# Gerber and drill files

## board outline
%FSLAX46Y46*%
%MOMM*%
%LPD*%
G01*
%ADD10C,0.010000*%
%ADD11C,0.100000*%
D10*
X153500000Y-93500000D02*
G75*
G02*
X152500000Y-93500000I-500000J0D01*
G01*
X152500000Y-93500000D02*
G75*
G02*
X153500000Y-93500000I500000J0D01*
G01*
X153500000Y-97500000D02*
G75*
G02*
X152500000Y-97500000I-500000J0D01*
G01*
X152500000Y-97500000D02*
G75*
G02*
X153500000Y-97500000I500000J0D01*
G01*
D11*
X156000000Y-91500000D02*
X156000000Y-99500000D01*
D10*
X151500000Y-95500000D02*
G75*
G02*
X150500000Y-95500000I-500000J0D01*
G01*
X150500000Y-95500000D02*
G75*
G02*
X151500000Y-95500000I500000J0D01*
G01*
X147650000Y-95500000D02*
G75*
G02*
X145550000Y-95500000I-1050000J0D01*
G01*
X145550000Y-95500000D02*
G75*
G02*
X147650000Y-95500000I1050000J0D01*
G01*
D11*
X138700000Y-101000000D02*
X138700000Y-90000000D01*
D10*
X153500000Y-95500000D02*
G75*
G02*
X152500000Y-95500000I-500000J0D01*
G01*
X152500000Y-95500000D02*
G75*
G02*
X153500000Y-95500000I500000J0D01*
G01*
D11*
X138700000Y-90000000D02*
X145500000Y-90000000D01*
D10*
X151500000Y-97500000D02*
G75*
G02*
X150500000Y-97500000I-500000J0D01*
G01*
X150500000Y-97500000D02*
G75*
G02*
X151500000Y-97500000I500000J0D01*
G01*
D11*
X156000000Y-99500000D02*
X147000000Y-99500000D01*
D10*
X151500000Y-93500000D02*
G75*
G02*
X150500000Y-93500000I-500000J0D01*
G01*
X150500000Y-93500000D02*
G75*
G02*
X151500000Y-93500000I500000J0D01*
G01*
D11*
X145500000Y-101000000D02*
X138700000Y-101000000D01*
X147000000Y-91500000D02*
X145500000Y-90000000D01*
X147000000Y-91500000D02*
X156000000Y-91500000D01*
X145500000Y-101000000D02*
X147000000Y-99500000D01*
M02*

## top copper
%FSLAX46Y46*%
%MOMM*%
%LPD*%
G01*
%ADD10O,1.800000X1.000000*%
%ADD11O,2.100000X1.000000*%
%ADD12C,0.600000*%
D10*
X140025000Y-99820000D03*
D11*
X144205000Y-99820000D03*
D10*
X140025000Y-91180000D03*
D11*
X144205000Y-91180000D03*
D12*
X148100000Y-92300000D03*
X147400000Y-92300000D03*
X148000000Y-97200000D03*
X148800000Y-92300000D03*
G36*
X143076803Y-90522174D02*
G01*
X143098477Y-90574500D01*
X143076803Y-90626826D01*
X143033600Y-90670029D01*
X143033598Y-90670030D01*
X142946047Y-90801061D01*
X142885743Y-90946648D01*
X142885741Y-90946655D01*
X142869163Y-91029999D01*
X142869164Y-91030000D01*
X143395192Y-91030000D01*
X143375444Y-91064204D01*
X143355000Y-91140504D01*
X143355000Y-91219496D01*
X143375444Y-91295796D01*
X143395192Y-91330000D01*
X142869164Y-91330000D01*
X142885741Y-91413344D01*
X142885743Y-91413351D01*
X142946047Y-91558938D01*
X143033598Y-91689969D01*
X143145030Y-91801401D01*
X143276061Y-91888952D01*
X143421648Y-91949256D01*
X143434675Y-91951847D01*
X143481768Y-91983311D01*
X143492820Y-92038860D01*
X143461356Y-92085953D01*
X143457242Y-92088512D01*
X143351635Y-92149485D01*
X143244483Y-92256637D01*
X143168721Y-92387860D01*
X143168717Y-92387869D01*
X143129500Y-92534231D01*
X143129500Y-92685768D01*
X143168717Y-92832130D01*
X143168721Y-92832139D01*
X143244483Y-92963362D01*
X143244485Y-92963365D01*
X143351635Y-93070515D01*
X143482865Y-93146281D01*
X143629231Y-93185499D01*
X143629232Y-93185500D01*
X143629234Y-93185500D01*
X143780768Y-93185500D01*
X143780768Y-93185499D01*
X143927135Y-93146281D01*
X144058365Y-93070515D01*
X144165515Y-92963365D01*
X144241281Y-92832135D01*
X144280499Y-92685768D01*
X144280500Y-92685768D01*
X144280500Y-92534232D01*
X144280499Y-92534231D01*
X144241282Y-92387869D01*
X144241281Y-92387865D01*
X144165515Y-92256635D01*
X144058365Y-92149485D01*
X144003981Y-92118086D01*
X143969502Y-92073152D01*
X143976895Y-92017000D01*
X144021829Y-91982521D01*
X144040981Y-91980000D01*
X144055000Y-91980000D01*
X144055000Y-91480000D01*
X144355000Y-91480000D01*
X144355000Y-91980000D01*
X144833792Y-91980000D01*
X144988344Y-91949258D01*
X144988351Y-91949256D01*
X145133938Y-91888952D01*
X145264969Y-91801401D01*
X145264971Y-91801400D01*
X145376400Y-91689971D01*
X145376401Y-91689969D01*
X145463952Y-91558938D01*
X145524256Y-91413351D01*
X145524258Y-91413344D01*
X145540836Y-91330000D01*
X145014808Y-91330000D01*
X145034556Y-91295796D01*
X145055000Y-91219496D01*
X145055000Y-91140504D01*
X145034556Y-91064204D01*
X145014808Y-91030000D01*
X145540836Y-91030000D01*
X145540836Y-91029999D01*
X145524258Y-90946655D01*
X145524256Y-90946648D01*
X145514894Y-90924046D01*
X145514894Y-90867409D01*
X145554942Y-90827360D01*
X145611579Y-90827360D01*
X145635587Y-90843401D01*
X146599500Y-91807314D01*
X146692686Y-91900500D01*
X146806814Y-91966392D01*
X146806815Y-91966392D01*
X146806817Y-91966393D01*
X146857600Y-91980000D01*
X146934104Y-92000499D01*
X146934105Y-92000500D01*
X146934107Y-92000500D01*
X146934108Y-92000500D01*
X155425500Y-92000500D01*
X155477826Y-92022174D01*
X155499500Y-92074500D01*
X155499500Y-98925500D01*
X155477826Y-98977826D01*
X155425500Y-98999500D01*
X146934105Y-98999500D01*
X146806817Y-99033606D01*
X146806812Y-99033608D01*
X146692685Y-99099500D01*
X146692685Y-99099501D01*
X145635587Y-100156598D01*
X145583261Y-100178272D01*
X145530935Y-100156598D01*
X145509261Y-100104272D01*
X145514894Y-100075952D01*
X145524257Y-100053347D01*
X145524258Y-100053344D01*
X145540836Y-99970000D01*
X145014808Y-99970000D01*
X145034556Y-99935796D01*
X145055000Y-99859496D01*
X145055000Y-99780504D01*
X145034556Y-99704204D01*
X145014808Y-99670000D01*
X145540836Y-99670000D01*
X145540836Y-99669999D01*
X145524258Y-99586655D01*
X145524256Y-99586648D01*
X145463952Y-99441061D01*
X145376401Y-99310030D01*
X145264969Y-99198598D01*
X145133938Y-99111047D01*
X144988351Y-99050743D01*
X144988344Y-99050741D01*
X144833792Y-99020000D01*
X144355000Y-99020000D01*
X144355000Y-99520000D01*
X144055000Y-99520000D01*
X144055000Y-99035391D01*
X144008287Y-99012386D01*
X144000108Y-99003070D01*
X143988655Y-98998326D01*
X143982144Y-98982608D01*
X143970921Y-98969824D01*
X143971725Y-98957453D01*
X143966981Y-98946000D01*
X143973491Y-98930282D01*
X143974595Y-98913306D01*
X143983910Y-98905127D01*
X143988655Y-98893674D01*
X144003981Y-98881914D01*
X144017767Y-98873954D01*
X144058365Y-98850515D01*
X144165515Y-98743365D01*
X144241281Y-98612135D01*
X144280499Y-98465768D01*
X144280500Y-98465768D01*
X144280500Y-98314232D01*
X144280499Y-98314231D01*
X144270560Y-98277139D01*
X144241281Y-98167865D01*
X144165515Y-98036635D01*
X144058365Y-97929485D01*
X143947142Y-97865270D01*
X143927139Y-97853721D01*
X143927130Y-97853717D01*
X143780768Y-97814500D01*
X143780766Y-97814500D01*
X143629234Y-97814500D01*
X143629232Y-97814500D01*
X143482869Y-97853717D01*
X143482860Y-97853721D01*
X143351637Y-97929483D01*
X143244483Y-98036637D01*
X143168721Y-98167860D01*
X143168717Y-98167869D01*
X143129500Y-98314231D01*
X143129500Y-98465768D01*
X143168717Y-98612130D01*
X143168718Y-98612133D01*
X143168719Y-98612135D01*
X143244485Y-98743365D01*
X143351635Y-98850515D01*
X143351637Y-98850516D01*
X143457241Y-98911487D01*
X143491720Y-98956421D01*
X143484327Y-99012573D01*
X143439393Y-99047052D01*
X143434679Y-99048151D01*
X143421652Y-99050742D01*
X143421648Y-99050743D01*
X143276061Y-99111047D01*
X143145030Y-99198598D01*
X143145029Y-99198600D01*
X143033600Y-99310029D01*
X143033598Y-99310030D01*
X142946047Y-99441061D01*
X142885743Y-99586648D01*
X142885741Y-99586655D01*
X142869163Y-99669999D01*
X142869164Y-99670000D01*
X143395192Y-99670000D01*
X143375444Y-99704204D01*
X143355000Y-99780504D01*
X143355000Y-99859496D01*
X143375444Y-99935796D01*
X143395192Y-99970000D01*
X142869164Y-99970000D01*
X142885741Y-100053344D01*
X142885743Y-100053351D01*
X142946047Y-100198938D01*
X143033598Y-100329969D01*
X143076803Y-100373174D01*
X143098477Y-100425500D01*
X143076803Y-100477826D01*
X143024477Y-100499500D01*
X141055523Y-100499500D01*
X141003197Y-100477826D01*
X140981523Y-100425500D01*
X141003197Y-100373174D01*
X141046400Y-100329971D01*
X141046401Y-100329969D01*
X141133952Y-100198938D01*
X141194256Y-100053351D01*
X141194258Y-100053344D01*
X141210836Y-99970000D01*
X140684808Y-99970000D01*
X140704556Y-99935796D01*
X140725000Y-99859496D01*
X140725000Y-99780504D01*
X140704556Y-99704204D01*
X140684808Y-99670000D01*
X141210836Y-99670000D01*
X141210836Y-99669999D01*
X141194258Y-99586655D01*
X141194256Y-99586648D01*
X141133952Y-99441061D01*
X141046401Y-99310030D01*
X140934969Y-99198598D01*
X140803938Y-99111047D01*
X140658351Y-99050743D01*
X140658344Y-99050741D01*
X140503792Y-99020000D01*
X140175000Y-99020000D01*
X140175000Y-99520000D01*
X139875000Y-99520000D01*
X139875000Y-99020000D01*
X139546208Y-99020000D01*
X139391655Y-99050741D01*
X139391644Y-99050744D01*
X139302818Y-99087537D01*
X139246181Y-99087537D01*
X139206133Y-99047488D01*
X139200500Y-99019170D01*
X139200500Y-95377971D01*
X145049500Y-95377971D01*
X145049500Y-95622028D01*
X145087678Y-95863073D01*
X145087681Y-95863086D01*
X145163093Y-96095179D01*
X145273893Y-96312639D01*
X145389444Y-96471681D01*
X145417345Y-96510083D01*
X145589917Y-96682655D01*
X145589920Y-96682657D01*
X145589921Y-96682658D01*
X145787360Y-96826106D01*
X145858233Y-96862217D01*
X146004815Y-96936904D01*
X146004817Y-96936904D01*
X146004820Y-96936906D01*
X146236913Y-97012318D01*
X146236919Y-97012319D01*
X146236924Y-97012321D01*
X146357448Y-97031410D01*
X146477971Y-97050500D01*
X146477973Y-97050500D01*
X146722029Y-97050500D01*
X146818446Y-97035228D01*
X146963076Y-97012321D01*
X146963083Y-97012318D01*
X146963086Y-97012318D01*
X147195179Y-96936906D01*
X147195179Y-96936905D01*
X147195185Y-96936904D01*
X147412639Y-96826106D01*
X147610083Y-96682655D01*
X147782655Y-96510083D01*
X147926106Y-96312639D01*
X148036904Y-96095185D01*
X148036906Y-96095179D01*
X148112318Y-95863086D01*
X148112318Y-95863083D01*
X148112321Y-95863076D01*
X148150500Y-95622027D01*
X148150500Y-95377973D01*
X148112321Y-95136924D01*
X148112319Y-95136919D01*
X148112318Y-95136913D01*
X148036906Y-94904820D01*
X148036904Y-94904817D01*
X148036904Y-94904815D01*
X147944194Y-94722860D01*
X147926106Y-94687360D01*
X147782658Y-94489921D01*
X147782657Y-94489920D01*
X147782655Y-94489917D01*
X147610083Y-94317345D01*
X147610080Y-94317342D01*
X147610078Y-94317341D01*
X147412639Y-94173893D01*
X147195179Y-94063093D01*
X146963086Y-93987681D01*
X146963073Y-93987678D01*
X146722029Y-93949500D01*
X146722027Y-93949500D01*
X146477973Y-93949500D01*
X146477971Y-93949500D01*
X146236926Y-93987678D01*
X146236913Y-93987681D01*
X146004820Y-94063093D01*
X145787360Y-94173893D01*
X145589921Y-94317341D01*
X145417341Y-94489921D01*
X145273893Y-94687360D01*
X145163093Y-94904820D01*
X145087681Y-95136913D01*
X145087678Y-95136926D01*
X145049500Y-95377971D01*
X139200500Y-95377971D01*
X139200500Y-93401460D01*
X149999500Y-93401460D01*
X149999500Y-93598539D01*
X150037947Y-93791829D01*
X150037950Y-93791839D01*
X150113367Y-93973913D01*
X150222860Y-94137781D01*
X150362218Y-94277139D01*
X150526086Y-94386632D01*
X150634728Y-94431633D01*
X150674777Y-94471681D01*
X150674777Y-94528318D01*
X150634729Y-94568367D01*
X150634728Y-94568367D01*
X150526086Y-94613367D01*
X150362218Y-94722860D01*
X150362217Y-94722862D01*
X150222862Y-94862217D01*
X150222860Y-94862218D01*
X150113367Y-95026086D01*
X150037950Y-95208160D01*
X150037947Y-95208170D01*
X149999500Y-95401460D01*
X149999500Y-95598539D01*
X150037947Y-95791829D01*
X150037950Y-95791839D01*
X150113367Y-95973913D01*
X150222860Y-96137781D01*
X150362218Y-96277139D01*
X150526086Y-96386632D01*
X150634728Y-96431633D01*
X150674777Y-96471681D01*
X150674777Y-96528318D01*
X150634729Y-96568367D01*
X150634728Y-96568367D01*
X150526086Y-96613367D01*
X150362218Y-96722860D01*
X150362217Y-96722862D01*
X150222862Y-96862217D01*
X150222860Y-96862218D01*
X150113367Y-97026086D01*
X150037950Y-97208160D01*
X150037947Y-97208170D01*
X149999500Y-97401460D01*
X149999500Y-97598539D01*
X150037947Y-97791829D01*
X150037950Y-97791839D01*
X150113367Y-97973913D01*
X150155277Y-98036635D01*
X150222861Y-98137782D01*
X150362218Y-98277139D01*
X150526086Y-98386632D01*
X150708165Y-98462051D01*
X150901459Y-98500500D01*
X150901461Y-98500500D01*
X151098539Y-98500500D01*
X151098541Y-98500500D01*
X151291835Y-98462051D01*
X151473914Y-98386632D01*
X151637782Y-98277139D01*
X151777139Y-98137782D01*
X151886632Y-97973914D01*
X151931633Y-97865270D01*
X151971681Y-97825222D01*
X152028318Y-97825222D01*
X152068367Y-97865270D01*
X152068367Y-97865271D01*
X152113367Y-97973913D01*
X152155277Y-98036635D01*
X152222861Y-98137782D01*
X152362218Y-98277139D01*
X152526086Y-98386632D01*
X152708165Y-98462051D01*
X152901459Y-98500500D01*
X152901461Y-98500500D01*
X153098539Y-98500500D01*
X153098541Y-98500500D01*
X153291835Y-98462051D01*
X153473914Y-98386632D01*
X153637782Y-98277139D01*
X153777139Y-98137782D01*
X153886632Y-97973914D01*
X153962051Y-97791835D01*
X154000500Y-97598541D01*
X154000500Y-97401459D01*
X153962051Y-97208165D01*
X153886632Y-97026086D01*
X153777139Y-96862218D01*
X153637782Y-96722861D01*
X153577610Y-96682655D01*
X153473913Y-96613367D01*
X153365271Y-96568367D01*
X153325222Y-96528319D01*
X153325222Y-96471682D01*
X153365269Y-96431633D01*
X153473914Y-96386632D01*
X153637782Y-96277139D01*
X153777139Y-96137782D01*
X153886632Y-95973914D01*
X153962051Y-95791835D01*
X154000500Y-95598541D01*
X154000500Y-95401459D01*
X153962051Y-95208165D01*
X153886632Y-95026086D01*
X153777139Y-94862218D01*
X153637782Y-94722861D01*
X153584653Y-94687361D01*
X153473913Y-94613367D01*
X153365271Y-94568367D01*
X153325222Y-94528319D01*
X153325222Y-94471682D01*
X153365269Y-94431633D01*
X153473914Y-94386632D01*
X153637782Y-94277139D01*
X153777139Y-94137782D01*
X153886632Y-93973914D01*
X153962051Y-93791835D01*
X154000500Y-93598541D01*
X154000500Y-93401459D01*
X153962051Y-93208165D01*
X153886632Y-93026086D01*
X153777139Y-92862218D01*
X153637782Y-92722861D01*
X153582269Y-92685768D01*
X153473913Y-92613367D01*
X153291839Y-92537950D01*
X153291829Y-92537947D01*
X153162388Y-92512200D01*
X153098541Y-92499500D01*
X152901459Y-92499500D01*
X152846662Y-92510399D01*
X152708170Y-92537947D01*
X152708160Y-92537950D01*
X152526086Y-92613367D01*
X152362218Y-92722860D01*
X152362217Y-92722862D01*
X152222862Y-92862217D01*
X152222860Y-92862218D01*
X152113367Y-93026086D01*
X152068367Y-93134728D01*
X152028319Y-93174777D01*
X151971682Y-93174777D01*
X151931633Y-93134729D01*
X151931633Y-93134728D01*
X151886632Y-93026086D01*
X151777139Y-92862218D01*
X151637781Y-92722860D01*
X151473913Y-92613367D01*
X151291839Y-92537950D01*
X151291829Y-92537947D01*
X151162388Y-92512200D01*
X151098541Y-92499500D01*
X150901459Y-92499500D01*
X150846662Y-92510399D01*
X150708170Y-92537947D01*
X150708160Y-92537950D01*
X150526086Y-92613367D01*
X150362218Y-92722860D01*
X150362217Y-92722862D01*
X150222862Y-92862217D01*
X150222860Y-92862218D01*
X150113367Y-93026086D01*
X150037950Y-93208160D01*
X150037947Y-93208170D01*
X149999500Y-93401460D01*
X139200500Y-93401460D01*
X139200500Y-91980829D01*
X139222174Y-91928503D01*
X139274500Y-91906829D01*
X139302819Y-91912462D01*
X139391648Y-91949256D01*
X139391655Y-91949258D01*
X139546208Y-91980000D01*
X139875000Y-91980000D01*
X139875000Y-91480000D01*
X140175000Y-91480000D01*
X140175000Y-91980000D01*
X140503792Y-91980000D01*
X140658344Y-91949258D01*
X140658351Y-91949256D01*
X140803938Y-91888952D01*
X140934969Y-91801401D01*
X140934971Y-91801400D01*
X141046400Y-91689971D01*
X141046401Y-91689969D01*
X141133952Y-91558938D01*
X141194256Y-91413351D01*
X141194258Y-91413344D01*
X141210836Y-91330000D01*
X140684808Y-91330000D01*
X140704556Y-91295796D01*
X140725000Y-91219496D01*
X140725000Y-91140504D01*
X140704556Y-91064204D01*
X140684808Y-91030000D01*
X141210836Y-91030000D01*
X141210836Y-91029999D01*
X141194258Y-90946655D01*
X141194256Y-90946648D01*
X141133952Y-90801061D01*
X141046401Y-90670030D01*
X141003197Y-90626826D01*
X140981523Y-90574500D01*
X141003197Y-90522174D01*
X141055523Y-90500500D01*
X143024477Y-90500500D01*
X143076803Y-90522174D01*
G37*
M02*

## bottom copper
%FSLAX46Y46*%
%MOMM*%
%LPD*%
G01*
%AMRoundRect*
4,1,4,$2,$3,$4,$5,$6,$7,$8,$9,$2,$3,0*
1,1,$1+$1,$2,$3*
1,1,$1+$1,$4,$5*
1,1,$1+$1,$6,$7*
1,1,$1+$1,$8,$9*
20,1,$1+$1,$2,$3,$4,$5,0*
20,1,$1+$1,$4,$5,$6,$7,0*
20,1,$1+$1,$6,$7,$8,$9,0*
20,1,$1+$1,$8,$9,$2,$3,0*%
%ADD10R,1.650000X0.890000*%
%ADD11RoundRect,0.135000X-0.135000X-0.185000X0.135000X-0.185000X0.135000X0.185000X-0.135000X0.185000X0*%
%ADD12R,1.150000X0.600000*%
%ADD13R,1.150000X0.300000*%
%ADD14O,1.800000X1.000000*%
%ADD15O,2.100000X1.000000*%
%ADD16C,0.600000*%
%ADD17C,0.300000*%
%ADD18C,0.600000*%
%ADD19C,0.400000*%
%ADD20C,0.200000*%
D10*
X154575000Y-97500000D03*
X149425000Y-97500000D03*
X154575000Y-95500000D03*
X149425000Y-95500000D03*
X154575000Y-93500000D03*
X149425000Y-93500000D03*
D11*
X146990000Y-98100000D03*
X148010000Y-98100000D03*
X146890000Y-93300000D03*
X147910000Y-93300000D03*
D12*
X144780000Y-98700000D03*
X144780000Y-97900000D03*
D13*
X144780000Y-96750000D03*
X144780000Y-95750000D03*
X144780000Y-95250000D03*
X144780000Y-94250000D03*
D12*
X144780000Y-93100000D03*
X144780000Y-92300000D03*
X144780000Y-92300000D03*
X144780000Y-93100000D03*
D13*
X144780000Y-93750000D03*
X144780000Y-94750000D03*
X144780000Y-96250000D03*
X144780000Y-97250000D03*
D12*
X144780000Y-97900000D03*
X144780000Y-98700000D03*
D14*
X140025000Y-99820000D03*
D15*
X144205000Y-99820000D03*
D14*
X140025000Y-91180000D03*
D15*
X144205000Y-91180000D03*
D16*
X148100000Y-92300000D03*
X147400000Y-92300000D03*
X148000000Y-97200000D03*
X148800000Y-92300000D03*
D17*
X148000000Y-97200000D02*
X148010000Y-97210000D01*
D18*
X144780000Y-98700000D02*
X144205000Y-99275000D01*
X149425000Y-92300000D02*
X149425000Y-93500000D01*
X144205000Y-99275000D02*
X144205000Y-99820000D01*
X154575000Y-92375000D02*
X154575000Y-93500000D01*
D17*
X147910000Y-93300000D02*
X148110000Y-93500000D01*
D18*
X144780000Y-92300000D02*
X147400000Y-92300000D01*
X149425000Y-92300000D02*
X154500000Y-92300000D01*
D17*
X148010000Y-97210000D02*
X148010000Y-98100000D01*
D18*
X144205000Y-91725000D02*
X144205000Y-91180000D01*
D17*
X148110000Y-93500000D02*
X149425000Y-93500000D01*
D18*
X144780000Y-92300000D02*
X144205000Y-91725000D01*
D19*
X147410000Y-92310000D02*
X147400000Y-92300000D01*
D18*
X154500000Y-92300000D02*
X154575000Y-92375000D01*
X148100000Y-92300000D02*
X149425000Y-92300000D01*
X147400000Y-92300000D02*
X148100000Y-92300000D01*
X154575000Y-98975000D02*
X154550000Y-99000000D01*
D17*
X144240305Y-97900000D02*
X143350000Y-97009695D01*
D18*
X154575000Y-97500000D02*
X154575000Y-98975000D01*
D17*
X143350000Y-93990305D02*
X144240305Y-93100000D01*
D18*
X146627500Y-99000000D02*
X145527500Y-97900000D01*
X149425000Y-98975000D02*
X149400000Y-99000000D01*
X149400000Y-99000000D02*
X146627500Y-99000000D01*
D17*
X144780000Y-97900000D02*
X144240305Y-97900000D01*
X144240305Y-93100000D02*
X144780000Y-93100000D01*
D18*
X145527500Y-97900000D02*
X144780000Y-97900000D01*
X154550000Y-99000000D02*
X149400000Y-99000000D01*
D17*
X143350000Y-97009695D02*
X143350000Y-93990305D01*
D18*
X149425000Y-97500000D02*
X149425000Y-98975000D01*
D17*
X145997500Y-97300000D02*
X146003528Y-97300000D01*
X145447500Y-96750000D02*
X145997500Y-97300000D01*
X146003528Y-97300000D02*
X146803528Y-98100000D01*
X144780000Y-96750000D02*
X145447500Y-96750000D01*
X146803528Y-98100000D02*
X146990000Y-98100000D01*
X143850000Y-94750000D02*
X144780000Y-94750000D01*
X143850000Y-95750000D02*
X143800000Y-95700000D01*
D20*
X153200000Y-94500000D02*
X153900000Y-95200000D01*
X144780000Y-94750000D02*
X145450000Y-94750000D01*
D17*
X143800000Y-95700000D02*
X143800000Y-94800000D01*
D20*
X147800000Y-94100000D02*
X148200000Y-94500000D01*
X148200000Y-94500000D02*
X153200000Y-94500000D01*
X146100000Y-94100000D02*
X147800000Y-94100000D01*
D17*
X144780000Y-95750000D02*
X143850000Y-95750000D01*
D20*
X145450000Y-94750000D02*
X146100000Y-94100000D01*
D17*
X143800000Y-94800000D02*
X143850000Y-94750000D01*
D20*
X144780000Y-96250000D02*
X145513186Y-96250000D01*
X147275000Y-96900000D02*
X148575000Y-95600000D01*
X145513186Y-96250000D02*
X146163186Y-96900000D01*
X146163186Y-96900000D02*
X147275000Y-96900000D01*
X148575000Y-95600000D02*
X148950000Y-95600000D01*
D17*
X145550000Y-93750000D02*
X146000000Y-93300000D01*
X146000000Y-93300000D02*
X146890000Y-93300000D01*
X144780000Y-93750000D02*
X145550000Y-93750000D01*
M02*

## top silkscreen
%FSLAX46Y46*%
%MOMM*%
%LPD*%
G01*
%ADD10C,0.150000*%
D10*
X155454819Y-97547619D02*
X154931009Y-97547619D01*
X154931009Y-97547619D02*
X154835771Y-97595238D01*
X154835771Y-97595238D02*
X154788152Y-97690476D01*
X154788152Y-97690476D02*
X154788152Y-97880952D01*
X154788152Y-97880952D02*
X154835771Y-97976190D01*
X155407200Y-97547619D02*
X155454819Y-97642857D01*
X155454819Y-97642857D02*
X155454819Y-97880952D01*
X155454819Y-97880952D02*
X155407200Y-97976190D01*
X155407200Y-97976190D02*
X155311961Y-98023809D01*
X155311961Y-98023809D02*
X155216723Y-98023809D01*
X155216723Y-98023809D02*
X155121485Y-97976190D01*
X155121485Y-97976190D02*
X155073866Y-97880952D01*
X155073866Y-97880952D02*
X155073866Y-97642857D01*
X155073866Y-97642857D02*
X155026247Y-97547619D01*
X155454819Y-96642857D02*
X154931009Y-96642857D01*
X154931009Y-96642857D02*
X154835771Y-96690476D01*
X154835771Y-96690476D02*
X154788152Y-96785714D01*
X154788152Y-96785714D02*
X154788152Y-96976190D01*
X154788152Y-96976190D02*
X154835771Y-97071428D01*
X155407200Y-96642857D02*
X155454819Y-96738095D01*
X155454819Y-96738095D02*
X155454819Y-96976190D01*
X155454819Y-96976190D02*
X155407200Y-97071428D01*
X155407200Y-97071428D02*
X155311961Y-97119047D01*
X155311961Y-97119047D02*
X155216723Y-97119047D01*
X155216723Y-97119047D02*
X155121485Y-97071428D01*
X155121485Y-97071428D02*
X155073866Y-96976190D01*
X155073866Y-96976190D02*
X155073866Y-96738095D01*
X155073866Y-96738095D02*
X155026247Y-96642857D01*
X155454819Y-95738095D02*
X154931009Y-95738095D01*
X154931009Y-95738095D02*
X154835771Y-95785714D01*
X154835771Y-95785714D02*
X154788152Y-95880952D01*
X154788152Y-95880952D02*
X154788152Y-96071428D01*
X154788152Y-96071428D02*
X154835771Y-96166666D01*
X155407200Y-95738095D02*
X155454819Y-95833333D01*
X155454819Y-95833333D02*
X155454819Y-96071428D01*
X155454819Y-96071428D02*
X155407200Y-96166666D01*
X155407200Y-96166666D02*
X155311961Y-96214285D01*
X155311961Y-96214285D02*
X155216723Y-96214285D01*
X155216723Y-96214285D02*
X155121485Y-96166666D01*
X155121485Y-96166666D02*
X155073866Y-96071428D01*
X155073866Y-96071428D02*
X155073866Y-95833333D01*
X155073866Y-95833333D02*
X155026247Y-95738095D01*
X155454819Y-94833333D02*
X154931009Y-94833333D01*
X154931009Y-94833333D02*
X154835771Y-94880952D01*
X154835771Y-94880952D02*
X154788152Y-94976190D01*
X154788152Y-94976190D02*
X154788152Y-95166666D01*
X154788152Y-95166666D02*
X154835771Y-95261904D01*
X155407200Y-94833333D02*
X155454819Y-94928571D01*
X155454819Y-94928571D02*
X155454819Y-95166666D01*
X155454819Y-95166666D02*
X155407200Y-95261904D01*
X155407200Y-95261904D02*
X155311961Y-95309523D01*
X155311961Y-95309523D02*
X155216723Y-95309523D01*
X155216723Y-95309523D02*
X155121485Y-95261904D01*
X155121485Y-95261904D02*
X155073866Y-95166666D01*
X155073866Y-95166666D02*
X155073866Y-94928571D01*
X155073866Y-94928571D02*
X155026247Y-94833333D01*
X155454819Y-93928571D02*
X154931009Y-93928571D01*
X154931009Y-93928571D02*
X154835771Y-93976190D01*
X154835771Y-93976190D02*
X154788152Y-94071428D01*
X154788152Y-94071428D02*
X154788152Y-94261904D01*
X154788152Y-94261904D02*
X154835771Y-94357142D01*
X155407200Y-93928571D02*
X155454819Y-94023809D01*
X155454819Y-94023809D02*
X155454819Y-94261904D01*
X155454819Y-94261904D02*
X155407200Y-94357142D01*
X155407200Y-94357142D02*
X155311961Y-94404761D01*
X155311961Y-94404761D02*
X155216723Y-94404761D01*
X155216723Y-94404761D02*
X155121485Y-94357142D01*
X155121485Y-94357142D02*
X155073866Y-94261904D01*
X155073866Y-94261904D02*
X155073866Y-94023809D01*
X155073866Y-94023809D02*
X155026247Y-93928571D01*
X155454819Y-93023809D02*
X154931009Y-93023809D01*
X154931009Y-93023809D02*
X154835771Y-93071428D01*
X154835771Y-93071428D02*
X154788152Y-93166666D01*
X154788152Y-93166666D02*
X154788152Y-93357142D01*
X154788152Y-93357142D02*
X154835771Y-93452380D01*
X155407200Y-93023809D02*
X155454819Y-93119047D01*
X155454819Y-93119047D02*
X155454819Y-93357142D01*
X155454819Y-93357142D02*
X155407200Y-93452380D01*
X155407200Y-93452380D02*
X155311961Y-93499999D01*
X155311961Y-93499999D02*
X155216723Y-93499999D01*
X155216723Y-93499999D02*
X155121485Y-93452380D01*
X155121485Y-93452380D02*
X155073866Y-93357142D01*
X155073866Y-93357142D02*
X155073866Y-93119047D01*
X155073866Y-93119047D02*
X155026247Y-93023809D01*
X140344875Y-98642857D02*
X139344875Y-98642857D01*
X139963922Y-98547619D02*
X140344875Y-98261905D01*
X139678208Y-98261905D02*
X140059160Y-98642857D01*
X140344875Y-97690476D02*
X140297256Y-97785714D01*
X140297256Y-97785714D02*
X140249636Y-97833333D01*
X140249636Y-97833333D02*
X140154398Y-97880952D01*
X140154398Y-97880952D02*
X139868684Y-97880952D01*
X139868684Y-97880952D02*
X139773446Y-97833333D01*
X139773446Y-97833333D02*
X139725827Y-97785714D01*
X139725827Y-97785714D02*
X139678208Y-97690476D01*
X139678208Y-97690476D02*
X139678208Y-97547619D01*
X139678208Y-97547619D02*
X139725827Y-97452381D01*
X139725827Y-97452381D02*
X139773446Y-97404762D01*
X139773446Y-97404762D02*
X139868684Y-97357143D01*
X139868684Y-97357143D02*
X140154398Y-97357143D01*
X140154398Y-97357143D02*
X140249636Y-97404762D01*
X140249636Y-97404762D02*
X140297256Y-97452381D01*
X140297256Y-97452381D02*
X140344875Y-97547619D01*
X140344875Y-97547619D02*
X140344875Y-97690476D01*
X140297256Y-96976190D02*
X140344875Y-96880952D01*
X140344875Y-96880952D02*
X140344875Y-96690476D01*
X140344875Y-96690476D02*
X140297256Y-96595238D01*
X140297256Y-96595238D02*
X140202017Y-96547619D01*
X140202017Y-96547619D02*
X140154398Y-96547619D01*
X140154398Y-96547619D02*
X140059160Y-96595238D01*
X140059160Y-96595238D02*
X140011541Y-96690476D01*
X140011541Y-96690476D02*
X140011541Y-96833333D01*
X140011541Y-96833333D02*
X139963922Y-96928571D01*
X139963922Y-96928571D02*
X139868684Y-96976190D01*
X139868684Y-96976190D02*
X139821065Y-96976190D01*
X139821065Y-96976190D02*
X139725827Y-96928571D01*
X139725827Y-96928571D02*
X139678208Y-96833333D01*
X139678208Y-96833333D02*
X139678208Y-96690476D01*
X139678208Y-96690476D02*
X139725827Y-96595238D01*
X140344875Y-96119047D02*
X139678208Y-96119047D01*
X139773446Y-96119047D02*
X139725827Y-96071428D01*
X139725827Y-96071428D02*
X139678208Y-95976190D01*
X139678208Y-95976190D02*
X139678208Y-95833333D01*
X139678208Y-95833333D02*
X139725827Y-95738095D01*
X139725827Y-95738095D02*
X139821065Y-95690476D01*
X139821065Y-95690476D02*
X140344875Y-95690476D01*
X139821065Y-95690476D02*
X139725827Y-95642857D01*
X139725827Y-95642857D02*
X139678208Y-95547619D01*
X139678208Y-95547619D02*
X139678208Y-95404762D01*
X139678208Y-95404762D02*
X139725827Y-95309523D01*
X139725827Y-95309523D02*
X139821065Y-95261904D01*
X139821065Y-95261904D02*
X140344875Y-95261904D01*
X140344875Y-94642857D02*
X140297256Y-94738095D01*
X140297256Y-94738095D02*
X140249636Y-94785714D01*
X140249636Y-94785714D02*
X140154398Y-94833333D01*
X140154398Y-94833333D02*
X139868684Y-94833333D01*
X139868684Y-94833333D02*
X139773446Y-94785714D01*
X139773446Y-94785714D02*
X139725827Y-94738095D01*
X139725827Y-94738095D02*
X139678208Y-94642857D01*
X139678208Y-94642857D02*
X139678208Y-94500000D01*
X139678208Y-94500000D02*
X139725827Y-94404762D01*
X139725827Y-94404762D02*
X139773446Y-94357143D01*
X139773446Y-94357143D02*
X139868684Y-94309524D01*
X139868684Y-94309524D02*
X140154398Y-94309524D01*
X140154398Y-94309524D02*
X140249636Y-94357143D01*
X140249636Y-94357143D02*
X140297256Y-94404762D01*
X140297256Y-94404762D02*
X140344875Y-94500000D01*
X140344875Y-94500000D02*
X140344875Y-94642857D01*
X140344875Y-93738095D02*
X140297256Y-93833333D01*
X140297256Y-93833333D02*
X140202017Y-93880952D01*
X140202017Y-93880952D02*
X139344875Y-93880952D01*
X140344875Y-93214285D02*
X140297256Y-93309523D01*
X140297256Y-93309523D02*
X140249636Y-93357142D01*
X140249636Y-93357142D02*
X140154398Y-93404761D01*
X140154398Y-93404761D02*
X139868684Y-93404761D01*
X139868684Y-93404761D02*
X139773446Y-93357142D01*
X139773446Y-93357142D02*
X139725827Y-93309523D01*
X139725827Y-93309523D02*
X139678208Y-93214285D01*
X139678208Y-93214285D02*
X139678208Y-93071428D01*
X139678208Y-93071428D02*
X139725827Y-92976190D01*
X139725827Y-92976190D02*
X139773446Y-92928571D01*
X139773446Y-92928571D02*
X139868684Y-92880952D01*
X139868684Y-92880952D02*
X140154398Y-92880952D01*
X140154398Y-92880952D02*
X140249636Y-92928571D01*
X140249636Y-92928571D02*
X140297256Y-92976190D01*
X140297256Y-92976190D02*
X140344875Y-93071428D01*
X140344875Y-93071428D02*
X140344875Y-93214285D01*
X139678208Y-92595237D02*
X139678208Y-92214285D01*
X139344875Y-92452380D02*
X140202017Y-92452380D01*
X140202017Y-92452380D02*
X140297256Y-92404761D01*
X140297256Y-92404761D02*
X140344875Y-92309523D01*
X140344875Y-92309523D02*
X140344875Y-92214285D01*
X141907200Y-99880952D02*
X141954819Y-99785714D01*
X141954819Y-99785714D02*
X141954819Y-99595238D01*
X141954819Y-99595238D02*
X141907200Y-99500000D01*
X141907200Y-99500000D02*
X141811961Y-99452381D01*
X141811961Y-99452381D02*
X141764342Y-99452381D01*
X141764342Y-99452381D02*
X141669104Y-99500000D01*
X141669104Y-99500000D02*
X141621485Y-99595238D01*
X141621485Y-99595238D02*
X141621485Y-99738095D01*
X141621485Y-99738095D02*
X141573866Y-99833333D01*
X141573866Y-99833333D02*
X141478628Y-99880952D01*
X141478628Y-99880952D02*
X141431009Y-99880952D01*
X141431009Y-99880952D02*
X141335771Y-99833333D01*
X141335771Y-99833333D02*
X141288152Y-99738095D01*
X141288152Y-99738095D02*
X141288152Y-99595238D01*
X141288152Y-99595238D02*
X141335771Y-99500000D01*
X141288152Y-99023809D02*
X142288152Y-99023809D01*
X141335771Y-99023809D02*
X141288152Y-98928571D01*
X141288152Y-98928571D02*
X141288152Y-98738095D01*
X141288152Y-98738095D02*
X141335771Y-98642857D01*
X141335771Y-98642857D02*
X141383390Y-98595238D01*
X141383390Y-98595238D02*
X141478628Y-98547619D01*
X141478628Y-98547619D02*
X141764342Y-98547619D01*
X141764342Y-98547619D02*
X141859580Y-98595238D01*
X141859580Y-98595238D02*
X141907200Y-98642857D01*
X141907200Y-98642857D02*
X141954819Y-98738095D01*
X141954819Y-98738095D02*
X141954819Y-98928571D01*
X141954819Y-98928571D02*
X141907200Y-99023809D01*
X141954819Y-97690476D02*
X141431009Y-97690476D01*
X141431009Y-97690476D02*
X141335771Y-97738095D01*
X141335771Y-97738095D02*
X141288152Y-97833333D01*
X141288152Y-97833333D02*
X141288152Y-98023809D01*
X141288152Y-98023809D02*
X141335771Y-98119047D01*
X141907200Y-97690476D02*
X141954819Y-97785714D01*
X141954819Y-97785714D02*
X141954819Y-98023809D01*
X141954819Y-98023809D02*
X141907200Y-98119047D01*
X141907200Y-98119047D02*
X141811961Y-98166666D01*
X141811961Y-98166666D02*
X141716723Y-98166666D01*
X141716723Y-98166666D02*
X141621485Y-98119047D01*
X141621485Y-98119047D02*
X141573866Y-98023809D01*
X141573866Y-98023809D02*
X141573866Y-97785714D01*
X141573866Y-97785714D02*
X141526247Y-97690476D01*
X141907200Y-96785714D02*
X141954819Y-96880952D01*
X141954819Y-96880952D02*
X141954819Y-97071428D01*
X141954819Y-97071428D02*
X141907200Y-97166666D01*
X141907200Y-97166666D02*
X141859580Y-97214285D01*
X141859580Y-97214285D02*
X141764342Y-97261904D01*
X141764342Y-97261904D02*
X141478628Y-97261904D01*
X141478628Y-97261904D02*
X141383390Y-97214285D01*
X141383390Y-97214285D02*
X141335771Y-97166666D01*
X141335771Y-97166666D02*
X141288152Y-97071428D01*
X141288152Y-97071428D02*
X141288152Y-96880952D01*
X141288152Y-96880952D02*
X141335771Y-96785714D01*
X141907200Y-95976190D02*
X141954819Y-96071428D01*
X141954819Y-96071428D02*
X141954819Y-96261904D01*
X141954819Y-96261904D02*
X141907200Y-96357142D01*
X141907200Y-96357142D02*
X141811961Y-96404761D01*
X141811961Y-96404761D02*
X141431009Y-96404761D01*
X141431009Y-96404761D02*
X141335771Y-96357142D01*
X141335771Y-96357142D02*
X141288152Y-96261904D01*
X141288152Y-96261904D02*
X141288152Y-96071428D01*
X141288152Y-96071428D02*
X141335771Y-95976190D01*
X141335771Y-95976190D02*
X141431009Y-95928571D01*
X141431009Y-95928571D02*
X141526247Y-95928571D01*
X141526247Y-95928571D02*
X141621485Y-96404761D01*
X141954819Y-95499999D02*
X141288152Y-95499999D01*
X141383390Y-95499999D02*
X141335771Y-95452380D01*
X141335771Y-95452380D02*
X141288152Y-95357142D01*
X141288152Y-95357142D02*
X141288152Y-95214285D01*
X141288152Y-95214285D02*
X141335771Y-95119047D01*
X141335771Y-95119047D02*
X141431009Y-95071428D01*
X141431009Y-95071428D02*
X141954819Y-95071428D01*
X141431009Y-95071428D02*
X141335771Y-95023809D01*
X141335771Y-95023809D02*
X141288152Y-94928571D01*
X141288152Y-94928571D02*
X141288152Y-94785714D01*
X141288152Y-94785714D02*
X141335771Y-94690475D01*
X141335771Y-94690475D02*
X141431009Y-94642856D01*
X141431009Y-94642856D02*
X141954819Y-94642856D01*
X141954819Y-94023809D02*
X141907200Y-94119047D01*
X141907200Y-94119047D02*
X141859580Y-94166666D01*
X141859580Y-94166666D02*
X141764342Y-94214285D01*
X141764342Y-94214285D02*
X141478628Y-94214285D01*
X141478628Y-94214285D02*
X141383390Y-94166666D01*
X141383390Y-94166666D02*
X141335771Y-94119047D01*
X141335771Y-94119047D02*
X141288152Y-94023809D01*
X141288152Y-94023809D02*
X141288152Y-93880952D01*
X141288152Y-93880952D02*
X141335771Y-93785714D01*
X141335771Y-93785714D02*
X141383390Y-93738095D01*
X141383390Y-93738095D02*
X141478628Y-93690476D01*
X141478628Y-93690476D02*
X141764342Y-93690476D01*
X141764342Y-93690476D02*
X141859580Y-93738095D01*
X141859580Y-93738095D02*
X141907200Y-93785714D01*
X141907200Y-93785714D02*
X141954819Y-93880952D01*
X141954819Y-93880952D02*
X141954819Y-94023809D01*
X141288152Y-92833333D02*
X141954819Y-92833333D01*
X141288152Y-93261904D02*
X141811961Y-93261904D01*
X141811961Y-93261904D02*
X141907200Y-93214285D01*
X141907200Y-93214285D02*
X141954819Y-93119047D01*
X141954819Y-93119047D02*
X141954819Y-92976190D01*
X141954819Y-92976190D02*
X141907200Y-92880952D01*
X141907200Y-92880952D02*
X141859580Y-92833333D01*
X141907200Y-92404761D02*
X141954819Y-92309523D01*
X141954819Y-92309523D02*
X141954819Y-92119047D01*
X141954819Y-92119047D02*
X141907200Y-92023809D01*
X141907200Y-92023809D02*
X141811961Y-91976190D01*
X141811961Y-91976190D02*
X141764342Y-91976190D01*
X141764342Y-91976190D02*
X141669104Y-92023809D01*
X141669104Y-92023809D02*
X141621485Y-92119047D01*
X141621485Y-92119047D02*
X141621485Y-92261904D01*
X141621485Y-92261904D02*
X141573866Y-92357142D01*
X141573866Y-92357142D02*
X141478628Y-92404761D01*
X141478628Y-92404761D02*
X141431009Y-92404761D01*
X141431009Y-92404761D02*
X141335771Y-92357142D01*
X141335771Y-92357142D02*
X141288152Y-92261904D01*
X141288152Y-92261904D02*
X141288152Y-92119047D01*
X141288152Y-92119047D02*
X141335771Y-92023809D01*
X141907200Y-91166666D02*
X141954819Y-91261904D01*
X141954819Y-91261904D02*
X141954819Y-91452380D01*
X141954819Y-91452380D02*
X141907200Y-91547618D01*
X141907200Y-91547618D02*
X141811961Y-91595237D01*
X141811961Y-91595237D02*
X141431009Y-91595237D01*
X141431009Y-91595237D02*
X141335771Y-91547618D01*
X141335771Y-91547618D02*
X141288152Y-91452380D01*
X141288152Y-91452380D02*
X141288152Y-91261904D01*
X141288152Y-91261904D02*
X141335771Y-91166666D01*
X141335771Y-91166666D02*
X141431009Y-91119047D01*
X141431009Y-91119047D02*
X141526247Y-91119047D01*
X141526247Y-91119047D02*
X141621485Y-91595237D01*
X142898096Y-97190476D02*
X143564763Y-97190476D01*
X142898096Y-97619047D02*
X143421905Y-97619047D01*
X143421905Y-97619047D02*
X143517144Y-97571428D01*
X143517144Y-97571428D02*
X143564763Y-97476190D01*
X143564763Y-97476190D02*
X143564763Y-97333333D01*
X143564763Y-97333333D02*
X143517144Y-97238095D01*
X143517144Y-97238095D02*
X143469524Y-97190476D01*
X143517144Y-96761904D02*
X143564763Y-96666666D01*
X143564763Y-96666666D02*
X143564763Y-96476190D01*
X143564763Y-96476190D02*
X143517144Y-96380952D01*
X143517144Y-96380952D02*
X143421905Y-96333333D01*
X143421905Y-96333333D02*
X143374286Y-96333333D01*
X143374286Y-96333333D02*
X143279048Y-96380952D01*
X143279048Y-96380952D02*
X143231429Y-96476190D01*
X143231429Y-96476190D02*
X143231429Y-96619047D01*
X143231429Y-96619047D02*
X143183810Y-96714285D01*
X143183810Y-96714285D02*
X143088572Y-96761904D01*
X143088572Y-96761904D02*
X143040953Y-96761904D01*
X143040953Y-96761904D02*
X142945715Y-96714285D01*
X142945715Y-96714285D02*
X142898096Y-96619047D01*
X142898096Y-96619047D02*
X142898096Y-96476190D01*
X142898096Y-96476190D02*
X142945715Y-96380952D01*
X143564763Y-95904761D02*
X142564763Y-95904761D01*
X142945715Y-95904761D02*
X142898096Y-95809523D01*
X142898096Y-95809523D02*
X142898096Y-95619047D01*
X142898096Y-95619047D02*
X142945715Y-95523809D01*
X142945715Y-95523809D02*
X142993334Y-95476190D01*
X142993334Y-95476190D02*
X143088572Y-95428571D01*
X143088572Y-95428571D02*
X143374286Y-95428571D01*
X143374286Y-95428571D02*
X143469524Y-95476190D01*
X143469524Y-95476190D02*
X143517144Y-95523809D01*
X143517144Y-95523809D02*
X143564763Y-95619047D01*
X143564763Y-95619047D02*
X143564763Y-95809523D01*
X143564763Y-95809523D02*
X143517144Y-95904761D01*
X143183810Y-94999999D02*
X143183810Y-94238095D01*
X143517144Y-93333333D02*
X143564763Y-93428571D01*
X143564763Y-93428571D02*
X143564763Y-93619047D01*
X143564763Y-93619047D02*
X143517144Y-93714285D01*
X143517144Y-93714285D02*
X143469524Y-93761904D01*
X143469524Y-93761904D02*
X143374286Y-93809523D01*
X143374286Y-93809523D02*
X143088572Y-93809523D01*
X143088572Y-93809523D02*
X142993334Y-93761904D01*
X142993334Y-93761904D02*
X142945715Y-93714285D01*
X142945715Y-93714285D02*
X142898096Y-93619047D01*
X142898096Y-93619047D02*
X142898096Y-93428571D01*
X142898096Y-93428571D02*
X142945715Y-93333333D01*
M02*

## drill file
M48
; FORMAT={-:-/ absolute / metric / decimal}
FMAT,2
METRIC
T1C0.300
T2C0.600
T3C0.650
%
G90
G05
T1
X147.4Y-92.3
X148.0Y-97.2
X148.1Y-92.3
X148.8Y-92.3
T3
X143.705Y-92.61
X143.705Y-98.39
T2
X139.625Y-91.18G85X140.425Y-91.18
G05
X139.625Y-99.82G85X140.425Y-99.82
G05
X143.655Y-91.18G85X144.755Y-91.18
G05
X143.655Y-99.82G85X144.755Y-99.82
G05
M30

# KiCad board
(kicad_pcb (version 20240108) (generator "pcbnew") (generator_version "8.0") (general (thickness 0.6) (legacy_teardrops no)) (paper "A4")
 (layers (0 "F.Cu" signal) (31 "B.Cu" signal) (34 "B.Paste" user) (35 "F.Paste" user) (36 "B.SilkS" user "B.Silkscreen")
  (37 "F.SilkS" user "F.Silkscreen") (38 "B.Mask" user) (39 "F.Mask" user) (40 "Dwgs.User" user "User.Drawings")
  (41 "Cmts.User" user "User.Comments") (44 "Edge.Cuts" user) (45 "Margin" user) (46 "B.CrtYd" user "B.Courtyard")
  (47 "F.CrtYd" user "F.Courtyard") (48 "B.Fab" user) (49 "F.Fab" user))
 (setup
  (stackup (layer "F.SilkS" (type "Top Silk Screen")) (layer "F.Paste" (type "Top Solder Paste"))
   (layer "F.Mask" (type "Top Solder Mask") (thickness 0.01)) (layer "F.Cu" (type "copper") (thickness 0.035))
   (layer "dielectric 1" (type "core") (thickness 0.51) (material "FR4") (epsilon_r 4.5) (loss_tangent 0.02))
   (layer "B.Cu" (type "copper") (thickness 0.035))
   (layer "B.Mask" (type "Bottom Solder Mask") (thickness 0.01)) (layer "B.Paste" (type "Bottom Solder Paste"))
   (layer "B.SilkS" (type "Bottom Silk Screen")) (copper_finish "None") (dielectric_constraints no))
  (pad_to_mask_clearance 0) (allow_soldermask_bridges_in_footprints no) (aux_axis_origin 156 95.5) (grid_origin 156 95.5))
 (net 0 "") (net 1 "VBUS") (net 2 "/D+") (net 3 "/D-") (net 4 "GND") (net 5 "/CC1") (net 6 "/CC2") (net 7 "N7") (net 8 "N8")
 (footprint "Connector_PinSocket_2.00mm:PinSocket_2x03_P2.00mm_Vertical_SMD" (layer "B.Cu") (at 152 95.5)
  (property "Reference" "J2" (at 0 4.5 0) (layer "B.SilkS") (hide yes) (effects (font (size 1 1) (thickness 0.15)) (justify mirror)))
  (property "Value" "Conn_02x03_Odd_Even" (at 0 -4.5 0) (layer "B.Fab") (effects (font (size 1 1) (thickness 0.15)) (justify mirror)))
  (pad "1" smd rect (at 2.575 2) (size 1.65 0.89) (layers "B.Cu" "B.Paste" "B.Mask") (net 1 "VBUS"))
  (pad "2" smd rect (at -2.575 2) (size 1.65 0.89) (layers "B.Cu" "B.Paste" "B.Mask") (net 1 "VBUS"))
  (pad "3" smd rect (at 2.575 0) (size 1.65 0.89) (layers "B.Cu" "B.Paste" "B.Mask") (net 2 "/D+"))
  (pad "4" smd rect (at -2.575 0) (size 1.65 0.89) (layers "B.Cu" "B.Paste" "B.Mask") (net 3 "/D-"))
  (pad "5" smd rect (at 2.575 -2) (size 1.65 0.89) (layers "B.Cu" "B.Paste" "B.Mask") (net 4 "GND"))
  (pad "6" smd rect (at -2.575 -2) (size 1.65 0.89) (layers "B.Cu" "B.Paste" "B.Mask") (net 4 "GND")))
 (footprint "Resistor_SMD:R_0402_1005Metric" (layer "B.Cu") (at 147.5 98.1)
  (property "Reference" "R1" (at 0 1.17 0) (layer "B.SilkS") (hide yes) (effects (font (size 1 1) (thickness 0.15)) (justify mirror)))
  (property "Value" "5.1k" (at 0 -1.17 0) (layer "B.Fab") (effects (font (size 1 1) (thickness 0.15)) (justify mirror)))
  (pad "1" smd roundrect (at -0.51 0) (size 0.54 0.64) (layers "B.Cu" "B.Paste" "B.Mask") (roundrect_rratio 0.25) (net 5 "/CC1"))
  (pad "2" smd roundrect (at 0.51 0) (size 0.54 0.64) (layers "B.Cu" "B.Paste" "B.Mask") (roundrect_rratio 0.25) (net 4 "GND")))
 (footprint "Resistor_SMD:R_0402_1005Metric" (layer "B.Cu") (at 147.4 93.3)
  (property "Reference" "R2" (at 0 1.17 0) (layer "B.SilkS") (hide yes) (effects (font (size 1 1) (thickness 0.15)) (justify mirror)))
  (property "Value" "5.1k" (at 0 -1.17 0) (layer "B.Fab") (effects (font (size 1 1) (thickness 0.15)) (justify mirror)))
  (pad "1" smd roundrect (at -0.51 0) (size 0.54 0.64) (layers "B.Cu" "B.Paste" "B.Mask") (roundrect_rratio 0.25) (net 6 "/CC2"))
  (pad "2" smd roundrect (at 0.51 0) (size 0.54 0.64) (layers "B.Cu" "B.Paste" "B.Mask") (roundrect_rratio 0.25) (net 4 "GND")))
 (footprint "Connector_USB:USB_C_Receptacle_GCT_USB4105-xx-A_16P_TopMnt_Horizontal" (layer "B.Cu") (at 141.1 95.5 90)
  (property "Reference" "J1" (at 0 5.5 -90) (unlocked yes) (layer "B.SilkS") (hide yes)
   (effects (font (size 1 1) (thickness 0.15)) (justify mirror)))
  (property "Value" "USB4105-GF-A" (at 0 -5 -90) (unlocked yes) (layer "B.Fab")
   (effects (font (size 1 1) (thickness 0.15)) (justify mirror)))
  (pad "" np_thru_hole circle (at -2.89 2.605 90) (size 0.65 0.65) (drill 0.65) (layers "F&B.Cu" "*.Mask"))
  (pad "" np_thru_hole circle (at 2.89 2.605 90) (size 0.65 0.65) (drill 0.65) (layers "F&B.Cu" "*.Mask"))
  (pad "A1" smd rect (at -3.2 3.68 90) (size 0.6 1.15) (layers "B.Cu" "B.Paste" "B.Mask") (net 4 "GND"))
  (pad "A4" smd rect (at -2.4 3.68 90) (size 0.6 1.15) (layers "B.Cu" "B.Paste" "B.Mask") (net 1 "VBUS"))
  (pad "A5" smd rect (at -1.25 3.68 90) (size 0.3 1.15) (layers "B.Cu" "B.Paste" "B.Mask") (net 5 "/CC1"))
  (pad "A6" smd rect (at -0.25 3.68 90) (size 0.3 1.15) (layers "B.Cu" "B.Paste" "B.Mask") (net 2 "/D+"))
  (pad "A7" smd rect (at 0.25 3.68 90) (size 0.3 1.15) (layers "B.Cu" "B.Paste" "B.Mask") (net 3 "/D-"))
  (pad "A8" smd rect (at 1.25 3.68 90) (size 0.3 1.15) (layers "B.Cu" "B.Paste" "B.Mask") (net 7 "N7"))
  (pad "A9" smd rect (at 2.4 3.68 90) (size 0.6 1.15) (layers "B.Cu" "B.Paste" "B.Mask") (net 1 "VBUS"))
  (pad "A12" smd rect (at 3.2 3.68 90) (size 0.6 1.15) (layers "B.Cu" "B.Paste" "B.Mask") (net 4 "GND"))
  (pad "B1" smd rect (at 3.2 3.68 90) (size 0.6 1.15) (layers "B.Cu" "B.Paste" "B.Mask") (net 4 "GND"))
  (pad "B4" smd rect (at 2.4 3.68 90) (size 0.6 1.15) (layers "B.Cu" "B.Paste" "B.Mask") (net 1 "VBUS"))
  (pad "B5" smd rect (at 1.75 3.68 90) (size 0.3 1.15) (layers "B.Cu" "B.Paste" "B.Mask") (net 6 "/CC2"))
  (pad "B6" smd rect (at 0.75 3.68 90) (size 0.3 1.15) (layers "B.Cu" "B.Paste" "B.Mask") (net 2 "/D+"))
  (pad "B7" smd rect (at -0.75 3.68 90) (size 0.3 1.15) (layers "B.Cu" "B.Paste" "B.Mask") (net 3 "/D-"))
  (pad "B8" smd rect (at -1.75 3.68 90) (size 0.3 1.15) (layers "B.Cu" "B.Paste" "B.Mask") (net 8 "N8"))
  (pad "B9" smd rect (at -2.4 3.68 90) (size 0.6 1.15) (layers "B.Cu" "B.Paste" "B.Mask") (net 1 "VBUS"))
  (pad "B12" smd rect (at -3.2 3.68 90) (size 0.6 1.15) (layers "B.Cu" "B.Paste" "B.Mask") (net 4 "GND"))
  (pad "S1" thru_hole oval (at -4.32 -1.075 90) (size 1 1.8) (drill oval 0.6 1.4) (layers "*.Cu" "*.Mask" "B.Paste")
   (remove_unused_layers no) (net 4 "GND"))
  (pad "S1" thru_hole oval (at -4.32 3.105 90) (size 1 2.1) (drill oval 0.6 1.7) (layers "*.Cu" "*.Mask" "B.Paste")
   (remove_unused_layers no) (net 4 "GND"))
  (pad "S1" thru_hole oval (at 4.32 -1.075 90) (size 1 1.8) (drill oval 0.6 1.4) (layers "*.Cu" "*.Mask" "B.Paste")
   (remove_unused_layers no) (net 4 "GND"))
  (pad "S1" thru_hole oval (at 4.32 3.105 90) (size 1 2.1) (drill oval 0.6 1.7) (layers "*.Cu" "*.Mask" "B.Paste") (remove_unused_layers no)
   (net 4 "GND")))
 (gr_circle (center 153 93.5) (end 153.5 93.5) (stroke (width 0.01) (type default)) (fill none) (layer "Edge.Cuts"))
 (gr_circle (center 153 97.5) (end 153.5 97.5) (stroke (width 0.01) (type default)) (fill none) (layer "Edge.Cuts"))
 (gr_line (start 156 91.5) (end 156 99.5) (stroke (width 0.1) (type default)) (layer "Edge.Cuts"))
 (gr_circle (center 151 95.5) (end 151.5 95.5) (stroke (width 0.01) (type default)) (fill none) (layer "Edge.Cuts"))
 (gr_circle (center 146.6 95.5) (end 147.65 95.5) (stroke (width 0.01) (type default)) (fill none) (layer "Edge.Cuts"))
 (gr_line (start 138.7 101) (end 138.7 90) (stroke (width 0.1) (type default)) (layer "Edge.Cuts"))
 (gr_circle (center 153 95.5) (end 153.5 95.5) (stroke (width 0.01) (type default)) (fill none) (layer "Edge.Cuts"))
 (gr_line (start 138.7 90) (end 145.5 90) (stroke (width 0.1) (type default)) (layer "Edge.Cuts"))
 (gr_circle (center 151 97.5) (end 151.5 97.5) (stroke (width 0.01) (type default)) (fill none) (layer "Edge.Cuts"))
 (gr_line (start 156 99.5) (end 147 99.5) (stroke (width 0.1) (type default)) (layer "Edge.Cuts"))
 (gr_circle (center 151 93.5) (end 151.5 93.5) (stroke (width 0.01) (type default)) (fill none) (layer "Edge.Cuts"))
 (gr_line (start 145.5 101) (end 138.7 101) (stroke (width 0.1) (type default)) (layer "Edge.Cuts"))
 (gr_line (start 147 91.5) (end 145.5 90) (stroke (width 0.1) (type default)) (layer "Edge.Cuts"))
 (gr_line (start 147 91.5) (end 156 91.5) (stroke (width 0.1) (type default)) (layer "Edge.Cuts"))
 (gr_line (start 145.5 101) (end 147 99.5) (stroke (width 0.1) (type default)) (layer "Edge.Cuts"))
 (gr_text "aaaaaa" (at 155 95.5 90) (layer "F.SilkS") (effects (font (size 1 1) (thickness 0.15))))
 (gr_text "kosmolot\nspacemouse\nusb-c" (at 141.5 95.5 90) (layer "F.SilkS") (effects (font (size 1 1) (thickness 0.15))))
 (via (at 148.1 92.3) (size 0.6) (drill 0.3) (layers "F.Cu" "B.Cu") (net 4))
 (via (at 147.4 92.3) (size 0.6) (drill 0.3) (layers "F.Cu" "B.Cu") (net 4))
 (via (at 148 97.2) (size 0.6) (drill 0.3) (layers "F.Cu" "B.Cu") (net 4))
 (via (at 148.8 92.3) (size 0.6) (drill 0.3) (layers "F.Cu" "B.Cu") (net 4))
 (segment (start 148 97.2) (end 148.01 97.21) (width 0.3) (layer "B.Cu") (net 4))
 (segment (start 144.78 98.7) (end 144.205 99.275) (width 0.6) (layer "B.Cu") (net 4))
 (segment (start 149.425 92.3) (end 149.425 93.5) (width 0.6) (layer "B.Cu") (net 4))
 (segment (start 144.205 99.275) (end 144.205 99.82) (width 0.6) (layer "B.Cu") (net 4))
 (segment (start 154.575 92.375) (end 154.575 93.5) (width 0.6) (layer "B.Cu") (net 4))
 (segment (start 147.91 93.3) (end 148.11 93.5) (width 0.3) (layer "B.Cu") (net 4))
 (segment (start 144.78 92.3) (end 147.4 92.3) (width 0.6) (layer "B.Cu") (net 4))
 (segment (start 149.425 92.3) (end 154.5 92.3) (width 0.6) (layer "B.Cu") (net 4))
 (segment (start 148.01 97.21) (end 148.01 98.1) (width 0.3) (layer "B.Cu") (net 4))
 (segment (start 144.205 91.725) (end 144.205 91.18) (width 0.6) (layer "B.Cu") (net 4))
 (segment (start 148.11 93.5) (end 149.425 93.5) (width 0.3) (layer "B.Cu") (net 4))
 (segment (start 144.78 92.3) (end 144.205 91.725) (width 0.6) (layer "B.Cu") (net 4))
 (segment (start 147.41 92.31) (end 147.4 92.3) (width 0.4) (layer "B.Cu") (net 4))
 (segment (start 154.5 92.3) (end 154.575 92.375) (width 0.6) (layer "B.Cu") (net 4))
 (segment (start 148.1 92.3) (end 149.425 92.3) (width 0.6) (layer "B.Cu") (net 4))
 (segment (start 147.4 92.3) (end 148.1 92.3) (width 0.6) (layer "B.Cu") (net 4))
 (segment (start 154.575 98.975) (end 154.55 99) (width 0.6) (layer "B.Cu") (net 1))
 (segment (start 144.240305 97.9) (end 143.35 97.009695) (width 0.3) (layer "B.Cu") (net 1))
 (segment (start 154.575 97.5) (end 154.575 98.975) (width 0.6) (layer "B.Cu") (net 1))
 (segment (start 143.35 93.990305) (end 144.240305 93.1) (width 0.3) (layer "B.Cu") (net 1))
 (segment (start 146.6275 99) (end 145.5275 97.9) (width 0.6) (layer "B.Cu") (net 1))
 (segment (start 149.425 98.975) (end 149.4 99) (width 0.6) (layer "B.Cu") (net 1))
 (segment (start 149.4 99) (end 146.6275 99) (width 0.6) (layer "B.Cu") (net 1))
 (segment (start 144.78 97.9) (end 144.240305 97.9) (width 0.3) (layer "B.Cu") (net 1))
 (segment (start 144.240305 93.1) (end 144.78 93.1) (width 0.3) (layer "B.Cu") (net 1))
 (segment (start 145.5275 97.9) (end 144.78 97.9) (width 0.6) (layer "B.Cu") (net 1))
 (segment (start 154.55 99) (end 149.4 99) (width 0.6) (layer "B.Cu") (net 1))
 (segment (start 143.35 97.009695) (end 143.35 93.990305) (width 0.3) (layer "B.Cu") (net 1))
 (segment (start 149.425 97.5) (end 149.425 98.975) (width 0.6) (layer "B.Cu") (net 1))
 (segment (start 145.9975 97.3) (end 146.003528 97.3) (width 0.3) (layer "B.Cu") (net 5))
 (segment (start 145.4475 96.75) (end 145.9975 97.3) (width 0.3) (layer "B.Cu") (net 5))
 (segment (start 146.003528 97.3) (end 146.803528 98.1) (width 0.3) (layer "B.Cu") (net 5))
 (segment (start 144.78 96.75) (end 145.4475 96.75) (width 0.3) (layer "B.Cu") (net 5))
 (segment (start 146.803528 98.1) (end 146.99 98.1) (width 0.3) (layer "B.Cu") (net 5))
 (segment (start 143.85 94.75) (end 144.78 94.75) (width 0.3) (layer "B.Cu") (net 2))
 (segment (start 143.85 95.75) (end 143.8 95.7) (width 0.3) (layer "B.Cu") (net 2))
 (segment (start 153.2 94.5) (end 153.9 95.2) (width 0.2) (layer "B.Cu") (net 2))
 (segment (start 144.78 94.75) (end 145.45 94.75) (width 0.2) (layer "B.Cu") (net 2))
 (segment (start 143.8 95.7) (end 143.8 94.8) (width 0.3) (layer "B.Cu") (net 2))
 (segment (start 147.8 94.1) (end 148.2 94.5) (width 0.2) (layer "B.Cu") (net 2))
 (segment (start 148.2 94.5) (end 153.2 94.5) (width 0.2) (layer "B.Cu") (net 2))
 (segment (start 146.1 94.1) (end 147.8 94.1) (width 0.2) (layer "B.Cu") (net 2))
 (segment (start 144.78 95.75) (end 143.85 95.75) (width 0.3) (layer "B.Cu") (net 2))
 (segment (start 145.45 94.75) (end 146.1 94.1) (width 0.2) (layer "B.Cu") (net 2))
 (segment (start 143.8 94.8) (end 143.85 94.75) (width 0.3) (layer "B.Cu") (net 2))
 (segment (start 144.78 96.25) (end 145.513186 96.25) (width 0.2) (layer "B.Cu") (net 3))
 (segment (start 147.275 96.9) (end 148.575 95.6) (width 0.2) (layer "B.Cu") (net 3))
 (segment (start 145.513186 96.25) (end 146.163186 96.9) (width 0.2) (layer "B.Cu") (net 3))
 (segment (start 146.163186 96.9) (end 147.275 96.9) (width 0.2) (layer "B.Cu") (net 3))
 (segment (start 148.575 95.6) (end 148.95 95.6) (width 0.2) (layer "B.Cu") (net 3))
 (segment (start 145.55 93.75) (end 146 93.3) (width 0.3) (layer "B.Cu") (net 6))
 (segment (start 146 93.3) (end 146.89 93.3) (width 0.3) (layer "B.Cu") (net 6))
 (segment (start 144.78 93.75) (end 145.55 93.75) (width 0.3) (layer "B.Cu") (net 6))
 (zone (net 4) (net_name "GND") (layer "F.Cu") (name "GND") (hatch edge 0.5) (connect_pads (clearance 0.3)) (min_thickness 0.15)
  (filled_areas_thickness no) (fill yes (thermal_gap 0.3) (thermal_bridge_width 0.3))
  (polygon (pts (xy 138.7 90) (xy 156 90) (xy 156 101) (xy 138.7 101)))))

